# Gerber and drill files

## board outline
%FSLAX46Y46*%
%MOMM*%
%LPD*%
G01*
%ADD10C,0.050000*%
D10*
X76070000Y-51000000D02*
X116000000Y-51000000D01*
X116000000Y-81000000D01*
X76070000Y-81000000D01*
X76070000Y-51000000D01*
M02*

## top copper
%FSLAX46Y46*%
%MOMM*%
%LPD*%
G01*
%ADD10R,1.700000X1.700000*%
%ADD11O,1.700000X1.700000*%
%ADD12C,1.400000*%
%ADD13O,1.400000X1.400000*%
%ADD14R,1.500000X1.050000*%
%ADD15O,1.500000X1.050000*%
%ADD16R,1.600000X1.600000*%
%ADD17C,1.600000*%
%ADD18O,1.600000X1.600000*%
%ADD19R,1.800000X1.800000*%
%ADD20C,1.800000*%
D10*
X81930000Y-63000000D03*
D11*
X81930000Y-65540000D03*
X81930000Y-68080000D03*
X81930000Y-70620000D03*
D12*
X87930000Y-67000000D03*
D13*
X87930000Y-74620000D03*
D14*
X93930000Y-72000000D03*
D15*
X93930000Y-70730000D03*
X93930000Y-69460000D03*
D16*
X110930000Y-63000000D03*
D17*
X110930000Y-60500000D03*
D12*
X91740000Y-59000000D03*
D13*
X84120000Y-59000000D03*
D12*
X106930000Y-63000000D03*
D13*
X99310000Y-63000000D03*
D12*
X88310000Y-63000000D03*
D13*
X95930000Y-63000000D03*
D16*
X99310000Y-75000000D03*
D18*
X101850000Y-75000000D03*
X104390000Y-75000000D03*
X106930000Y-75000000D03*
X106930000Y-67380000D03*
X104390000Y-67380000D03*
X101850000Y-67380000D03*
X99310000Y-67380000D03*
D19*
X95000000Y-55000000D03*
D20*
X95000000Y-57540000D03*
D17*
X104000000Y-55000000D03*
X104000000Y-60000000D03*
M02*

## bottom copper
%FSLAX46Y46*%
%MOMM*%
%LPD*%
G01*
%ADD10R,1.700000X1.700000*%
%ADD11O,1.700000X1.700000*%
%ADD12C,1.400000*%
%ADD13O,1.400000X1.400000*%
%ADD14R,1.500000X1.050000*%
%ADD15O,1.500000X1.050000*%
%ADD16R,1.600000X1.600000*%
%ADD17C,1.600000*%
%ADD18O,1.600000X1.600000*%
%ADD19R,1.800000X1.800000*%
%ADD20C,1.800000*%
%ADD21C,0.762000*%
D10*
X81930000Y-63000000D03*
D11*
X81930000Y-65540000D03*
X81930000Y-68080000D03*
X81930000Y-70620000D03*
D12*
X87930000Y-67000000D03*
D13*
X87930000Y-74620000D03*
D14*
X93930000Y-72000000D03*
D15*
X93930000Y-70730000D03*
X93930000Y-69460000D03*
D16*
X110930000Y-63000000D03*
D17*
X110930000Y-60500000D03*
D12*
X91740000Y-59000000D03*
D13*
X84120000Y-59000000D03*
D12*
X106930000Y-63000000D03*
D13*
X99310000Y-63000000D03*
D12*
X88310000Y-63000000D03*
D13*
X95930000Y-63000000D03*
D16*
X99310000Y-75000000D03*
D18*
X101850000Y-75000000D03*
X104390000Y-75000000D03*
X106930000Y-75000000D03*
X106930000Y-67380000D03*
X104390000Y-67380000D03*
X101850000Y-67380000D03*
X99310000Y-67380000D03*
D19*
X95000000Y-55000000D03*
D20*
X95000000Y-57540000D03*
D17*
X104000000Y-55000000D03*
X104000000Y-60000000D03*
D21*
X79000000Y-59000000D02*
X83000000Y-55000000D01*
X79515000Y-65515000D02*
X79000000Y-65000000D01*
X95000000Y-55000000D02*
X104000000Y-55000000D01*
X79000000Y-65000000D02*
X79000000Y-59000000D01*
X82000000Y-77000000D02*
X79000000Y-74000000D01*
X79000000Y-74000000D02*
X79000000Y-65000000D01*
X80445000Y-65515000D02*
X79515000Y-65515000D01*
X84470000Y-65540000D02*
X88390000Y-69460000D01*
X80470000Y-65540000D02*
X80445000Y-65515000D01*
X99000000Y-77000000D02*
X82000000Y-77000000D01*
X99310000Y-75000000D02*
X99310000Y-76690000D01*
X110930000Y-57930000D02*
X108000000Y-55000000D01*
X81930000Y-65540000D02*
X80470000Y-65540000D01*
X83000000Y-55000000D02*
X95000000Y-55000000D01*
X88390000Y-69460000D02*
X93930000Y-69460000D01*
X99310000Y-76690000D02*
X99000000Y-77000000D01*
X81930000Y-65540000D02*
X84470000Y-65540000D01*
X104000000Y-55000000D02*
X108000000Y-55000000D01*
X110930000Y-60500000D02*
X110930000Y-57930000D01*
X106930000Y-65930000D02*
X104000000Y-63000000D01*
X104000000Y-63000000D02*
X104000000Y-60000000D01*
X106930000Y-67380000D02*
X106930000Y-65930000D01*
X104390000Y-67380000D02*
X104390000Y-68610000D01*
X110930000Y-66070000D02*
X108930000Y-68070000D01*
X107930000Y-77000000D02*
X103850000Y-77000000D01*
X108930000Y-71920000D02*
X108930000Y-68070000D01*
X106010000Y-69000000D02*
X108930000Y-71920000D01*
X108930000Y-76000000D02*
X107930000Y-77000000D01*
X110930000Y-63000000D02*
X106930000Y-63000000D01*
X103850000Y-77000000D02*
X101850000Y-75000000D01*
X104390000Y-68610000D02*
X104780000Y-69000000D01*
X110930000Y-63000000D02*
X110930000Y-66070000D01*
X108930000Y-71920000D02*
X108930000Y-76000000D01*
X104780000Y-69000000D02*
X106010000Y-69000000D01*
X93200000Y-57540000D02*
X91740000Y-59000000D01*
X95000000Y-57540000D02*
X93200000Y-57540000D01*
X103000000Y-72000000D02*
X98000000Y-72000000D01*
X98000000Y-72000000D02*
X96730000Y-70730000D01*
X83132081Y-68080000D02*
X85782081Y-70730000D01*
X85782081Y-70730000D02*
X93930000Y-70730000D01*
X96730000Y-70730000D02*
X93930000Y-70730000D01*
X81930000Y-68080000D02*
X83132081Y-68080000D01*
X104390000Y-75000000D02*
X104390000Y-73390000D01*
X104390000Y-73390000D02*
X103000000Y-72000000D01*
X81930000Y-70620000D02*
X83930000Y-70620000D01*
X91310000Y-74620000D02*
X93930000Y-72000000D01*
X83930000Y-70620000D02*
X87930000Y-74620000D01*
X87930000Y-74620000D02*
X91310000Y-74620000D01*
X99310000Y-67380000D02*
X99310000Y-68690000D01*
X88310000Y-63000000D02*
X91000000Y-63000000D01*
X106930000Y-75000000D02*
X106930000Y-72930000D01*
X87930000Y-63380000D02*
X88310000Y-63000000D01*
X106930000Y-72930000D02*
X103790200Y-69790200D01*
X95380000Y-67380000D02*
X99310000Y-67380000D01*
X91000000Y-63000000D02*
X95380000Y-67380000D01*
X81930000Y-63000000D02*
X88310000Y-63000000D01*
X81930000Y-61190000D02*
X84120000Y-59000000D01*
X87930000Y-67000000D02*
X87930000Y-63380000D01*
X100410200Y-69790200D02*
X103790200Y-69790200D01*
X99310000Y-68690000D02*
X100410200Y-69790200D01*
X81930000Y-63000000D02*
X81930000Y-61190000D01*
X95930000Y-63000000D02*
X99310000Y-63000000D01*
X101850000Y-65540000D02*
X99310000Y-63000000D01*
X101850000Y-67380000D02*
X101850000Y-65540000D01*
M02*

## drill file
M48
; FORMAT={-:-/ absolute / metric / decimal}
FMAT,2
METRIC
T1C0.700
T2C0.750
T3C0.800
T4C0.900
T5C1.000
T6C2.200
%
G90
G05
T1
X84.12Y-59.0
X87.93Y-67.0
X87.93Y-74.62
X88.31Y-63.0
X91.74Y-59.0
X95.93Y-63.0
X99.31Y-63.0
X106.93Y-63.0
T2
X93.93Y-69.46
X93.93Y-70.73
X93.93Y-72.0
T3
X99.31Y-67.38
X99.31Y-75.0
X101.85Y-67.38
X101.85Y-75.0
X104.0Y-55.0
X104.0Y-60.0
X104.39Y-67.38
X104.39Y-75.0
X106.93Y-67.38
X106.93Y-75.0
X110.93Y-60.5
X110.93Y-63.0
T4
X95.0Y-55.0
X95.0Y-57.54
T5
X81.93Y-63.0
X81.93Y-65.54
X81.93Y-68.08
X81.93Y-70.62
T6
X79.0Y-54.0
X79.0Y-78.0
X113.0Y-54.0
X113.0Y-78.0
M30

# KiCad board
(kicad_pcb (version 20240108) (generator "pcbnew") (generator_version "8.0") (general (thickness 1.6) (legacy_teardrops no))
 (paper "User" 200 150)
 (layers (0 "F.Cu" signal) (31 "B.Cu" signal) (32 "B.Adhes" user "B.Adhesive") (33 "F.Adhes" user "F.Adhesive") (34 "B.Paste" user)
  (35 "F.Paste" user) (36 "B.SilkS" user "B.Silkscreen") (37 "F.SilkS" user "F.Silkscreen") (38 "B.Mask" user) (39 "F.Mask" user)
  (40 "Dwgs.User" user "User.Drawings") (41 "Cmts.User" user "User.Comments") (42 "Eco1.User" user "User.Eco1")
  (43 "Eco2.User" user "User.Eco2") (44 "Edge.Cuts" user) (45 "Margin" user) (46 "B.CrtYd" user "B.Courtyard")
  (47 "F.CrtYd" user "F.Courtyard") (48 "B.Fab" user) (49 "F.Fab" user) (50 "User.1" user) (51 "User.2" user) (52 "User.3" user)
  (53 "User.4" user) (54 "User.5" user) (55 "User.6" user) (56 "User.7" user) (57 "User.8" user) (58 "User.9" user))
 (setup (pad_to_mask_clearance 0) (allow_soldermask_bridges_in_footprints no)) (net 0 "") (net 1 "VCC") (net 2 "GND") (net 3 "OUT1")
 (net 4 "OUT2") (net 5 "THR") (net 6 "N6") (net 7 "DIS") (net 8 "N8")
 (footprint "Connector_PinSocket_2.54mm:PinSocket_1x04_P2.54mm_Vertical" (layer "F.Cu") (at 81.93 63)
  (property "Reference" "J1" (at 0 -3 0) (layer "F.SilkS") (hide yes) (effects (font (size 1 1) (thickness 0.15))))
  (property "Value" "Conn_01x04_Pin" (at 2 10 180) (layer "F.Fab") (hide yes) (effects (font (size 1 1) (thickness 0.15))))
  (pad "1" thru_hole rect (at 0 0) (size 1.7 1.7) (drill 1) (layers "*.Cu" "*.Mask") (remove_unused_layers no) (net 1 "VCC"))
  (pad "2" thru_hole oval (at 0 2.54) (size 1.7 1.7) (drill 1) (layers "*.Cu" "*.Mask") (remove_unused_layers no) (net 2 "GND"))
  (pad "3" thru_hole oval (at 0 5.08) (size 1.7 1.7) (drill 1) (layers "*.Cu" "*.Mask") (remove_unused_layers no) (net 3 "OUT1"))
  (pad "4" thru_hole oval (at 0 7.62) (size 1.7 1.7) (drill 1) (layers "*.Cu" "*.Mask") (remove_unused_layers no) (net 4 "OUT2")))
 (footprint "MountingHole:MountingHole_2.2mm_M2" (layer "F.Cu") (at 113 54)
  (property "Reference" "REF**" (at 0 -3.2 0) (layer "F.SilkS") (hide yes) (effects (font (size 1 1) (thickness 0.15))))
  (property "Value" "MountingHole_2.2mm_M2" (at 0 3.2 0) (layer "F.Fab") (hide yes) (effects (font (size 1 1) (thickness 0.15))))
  (pad "" np_thru_hole circle (at 0 0) (size 2.2 2.2) (drill 2.2) (layers "*.Cu" "*.Mask")))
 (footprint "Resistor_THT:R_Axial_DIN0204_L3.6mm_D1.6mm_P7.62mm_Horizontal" (layer "F.Cu") (at 87.93 67 -90)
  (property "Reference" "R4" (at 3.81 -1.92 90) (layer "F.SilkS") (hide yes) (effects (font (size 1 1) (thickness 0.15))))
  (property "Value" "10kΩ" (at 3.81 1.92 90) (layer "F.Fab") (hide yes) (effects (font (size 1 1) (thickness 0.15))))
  (pad "1" thru_hole circle (at 0 0 270) (size 1.4 1.4) (drill 0.7) (layers "*.Cu" "*.Mask") (remove_unused_layers no) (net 1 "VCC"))
  (pad "2" thru_hole oval (at 7.62 0 270) (size 1.4 1.4) (drill 0.7) (layers "*.Cu" "*.Mask") (remove_unused_layers no) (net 4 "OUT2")))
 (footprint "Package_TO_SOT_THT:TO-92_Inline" (layer "F.Cu") (at 93.93 72 90)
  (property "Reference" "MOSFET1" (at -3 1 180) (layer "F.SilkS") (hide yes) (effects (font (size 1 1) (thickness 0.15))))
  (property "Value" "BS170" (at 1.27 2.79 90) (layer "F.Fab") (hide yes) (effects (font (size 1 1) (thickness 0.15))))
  (pad "1" thru_hole rect (at 0 0 90) (size 1.05 1.5) (drill 0.75) (layers "*.Cu" "*.Mask") (remove_unused_layers no) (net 4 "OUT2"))
  (pad "2" thru_hole oval (at 1.27 0 90) (size 1.05 1.5) (drill 0.75) (layers "*.Cu" "*.Mask") (remove_unused_layers no) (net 3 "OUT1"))
  (pad "3" thru_hole oval (at 2.54 0 90) (size 1.05 1.5) (drill 0.75) (layers "*.Cu" "*.Mask") (remove_unused_layers no) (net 2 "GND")))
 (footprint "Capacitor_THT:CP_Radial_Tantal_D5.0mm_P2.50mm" (layer "F.Cu") (at 110.93 63 90)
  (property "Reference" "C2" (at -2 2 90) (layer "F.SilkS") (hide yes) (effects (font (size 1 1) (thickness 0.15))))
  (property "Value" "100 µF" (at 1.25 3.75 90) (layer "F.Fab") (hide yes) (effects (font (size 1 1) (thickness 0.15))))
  (pad "1" thru_hole rect (at 0 0 90) (size 1.6 1.6) (drill 0.8) (layers "*.Cu" "*.Mask") (remove_unused_layers no) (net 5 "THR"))
  (pad "2" thru_hole circle (at 2.5 0 90) (size 1.6 1.6) (drill 0.8) (layers "*.Cu" "*.Mask") (remove_unused_layers no) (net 2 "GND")))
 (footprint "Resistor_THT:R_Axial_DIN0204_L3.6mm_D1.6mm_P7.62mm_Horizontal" (layer "F.Cu") (at 91.74 59 180)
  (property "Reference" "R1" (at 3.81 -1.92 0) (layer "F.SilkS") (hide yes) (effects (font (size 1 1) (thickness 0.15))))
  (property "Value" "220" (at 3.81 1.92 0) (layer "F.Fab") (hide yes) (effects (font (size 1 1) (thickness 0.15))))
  (pad "1" thru_hole circle (at 0 0 180) (size 1.4 1.4) (drill 0.7) (layers "*.Cu" "*.Mask") (remove_unused_layers no) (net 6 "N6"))
  (pad "2" thru_hole oval (at 7.62 0 180) (size 1.4 1.4) (drill 0.7) (layers "*.Cu" "*.Mask") (remove_unused_layers no) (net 1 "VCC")))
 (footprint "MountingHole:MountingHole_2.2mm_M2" (layer "F.Cu") (at 113 78)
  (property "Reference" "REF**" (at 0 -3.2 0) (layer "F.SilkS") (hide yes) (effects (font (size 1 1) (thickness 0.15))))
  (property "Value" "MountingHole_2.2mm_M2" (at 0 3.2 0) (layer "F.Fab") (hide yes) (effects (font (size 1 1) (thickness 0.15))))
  (pad "" np_thru_hole circle (at 0 0) (size 2.2 2.2) (drill 2.2) (layers "*.Cu" "*.Mask")))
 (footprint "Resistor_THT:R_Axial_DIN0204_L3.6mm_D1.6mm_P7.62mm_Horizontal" (layer "F.Cu") (at 106.93 63 180)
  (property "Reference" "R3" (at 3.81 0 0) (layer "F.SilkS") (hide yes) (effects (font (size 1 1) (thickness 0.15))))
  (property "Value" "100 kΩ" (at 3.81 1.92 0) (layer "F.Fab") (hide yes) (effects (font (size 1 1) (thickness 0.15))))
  (pad "1" thru_hole circle (at 0 0 180) (size 1.4 1.4) (drill 0.7) (layers "*.Cu" "*.Mask") (remove_unused_layers no) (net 5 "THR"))
  (pad "2" thru_hole oval (at 7.62 0 180) (size 1.4 1.4) (drill 0.7) (layers "*.Cu" "*.Mask") (remove_unused_layers no) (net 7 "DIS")))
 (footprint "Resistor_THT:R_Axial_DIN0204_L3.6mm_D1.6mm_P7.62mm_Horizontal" (layer "F.Cu") (at 88.31 63)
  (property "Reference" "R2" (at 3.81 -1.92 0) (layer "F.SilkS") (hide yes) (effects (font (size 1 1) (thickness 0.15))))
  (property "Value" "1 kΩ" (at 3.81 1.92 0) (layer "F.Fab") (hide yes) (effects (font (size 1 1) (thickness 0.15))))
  (pad "1" thru_hole circle (at 0 0) (size 1.4 1.4) (drill 0.7) (layers "*.Cu" "*.Mask") (remove_unused_layers no) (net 1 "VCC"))
  (pad "2" thru_hole oval (at 7.62 0) (size 1.4 1.4) (drill 0.7) (layers "*.Cu" "*.Mask") (remove_unused_layers no) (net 7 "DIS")))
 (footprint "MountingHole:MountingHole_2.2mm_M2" (layer "F.Cu") (at 79 78)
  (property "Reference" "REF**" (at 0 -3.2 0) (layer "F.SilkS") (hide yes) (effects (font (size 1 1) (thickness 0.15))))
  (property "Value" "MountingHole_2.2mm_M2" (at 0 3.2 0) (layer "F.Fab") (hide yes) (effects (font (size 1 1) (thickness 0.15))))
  (pad "" np_thru_hole circle (at 0 0) (size 2.2 2.2) (drill 2.2) (layers "*.Cu" "*.Mask")))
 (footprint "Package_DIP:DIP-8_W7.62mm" (layer "F.Cu") (at 99.31 75 90)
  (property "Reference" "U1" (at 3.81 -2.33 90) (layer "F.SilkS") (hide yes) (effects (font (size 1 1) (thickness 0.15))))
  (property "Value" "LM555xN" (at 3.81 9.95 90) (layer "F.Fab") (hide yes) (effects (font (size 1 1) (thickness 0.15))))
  (pad "1" thru_hole rect (at 0 0 90) (size 1.6 1.6) (drill 0.8) (layers "*.Cu" "*.Mask") (remove_unused_layers no) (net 2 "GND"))
  (pad "2" thru_hole oval (at 0 2.54 90) (size 1.6 1.6) (drill 0.8) (layers "*.Cu" "*.Mask") (remove_unused_layers no) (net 5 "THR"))
  (pad "3" thru_hole oval (at 0 5.08 90) (size 1.6 1.6) (drill 0.8) (layers "*.Cu" "*.Mask") (remove_unused_layers no) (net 3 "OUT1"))
  (pad "4" thru_hole oval (at 0 7.62 90) (size 1.6 1.6) (drill 0.8) (layers "*.Cu" "*.Mask") (remove_unused_layers no) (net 1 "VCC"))
  (pad "5" thru_hole oval (at 7.62 7.62 90) (size 1.6 1.6) (drill 0.8) (layers "*.Cu" "*.Mask") (remove_unused_layers no) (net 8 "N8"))
  (pad "6" thru_hole oval (at 7.62 5.08 90) (size 1.6 1.6) (drill 0.8) (layers "*.Cu" "*.Mask") (remove_unused_layers no) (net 5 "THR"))
  (pad "7" thru_hole oval (at 7.62 2.54 90) (size 1.6 1.6) (drill 0.8) (layers "*.Cu" "*.Mask") (remove_unused_layers no) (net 7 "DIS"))
  (pad "8" thru_hole oval (at 7.62 0 90) (size 1.6 1.6) (drill 0.8) (layers "*.Cu" "*.Mask") (remove_unused_layers no) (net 1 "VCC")))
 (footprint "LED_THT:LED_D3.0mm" (layer "F.Cu") (at 95 55 -90)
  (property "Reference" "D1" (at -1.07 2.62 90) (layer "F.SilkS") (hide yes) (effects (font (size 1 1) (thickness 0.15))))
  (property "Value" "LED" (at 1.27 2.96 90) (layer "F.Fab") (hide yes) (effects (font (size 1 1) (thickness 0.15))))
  (pad "1" thru_hole rect (at 0 0 270) (size 1.8 1.8) (drill 0.9) (layers "*.Cu" "*.Mask") (remove_unused_layers no) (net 2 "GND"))
  (pad "2" thru_hole circle (at 2.54 0 270) (size 1.8 1.8) (drill 0.9) (layers "*.Cu" "*.Mask") (remove_unused_layers no) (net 6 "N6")))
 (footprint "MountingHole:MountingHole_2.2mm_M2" (layer "F.Cu") (at 79 54)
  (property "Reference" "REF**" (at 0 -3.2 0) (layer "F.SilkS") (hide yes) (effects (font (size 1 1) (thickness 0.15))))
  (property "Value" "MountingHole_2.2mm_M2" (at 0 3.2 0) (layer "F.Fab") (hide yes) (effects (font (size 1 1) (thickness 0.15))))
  (pad "" np_thru_hole circle (at 0 0) (size 2.2 2.2) (drill 2.2) (layers "*.Cu" "*.Mask")))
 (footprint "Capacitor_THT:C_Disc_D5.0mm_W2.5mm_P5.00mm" (layer "F.Cu") (at 104 55 -90)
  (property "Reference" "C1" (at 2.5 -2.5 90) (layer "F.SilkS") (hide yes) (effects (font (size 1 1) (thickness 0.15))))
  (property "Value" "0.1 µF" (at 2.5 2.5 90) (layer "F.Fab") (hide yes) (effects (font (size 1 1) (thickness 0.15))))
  (pad "1" thru_hole circle (at 0 0 270) (size 1.6 1.6) (drill 0.8) (layers "*.Cu" "*.Mask") (remove_unused_layers no) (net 2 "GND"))
  (pad "2" thru_hole circle (at 5 0 270) (size 1.6 1.6) (drill 0.8) (layers "*.Cu" "*.Mask") (remove_unused_layers no) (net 8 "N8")))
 (gr_rect (start 76.07 51) (end 116 81) (stroke (width 0.05) (type default)) (fill none) (layer "Edge.Cuts"))
 (segment (start 79 59) (end 83 55) (width 0.762) (layer "B.Cu") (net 2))
 (segment (start 79.515 65.515) (end 79 65) (width 0.762) (layer "B.Cu") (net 2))
 (segment (start 95 55) (end 104 55) (width 0.762) (layer "B.Cu") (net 2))
 (segment (start 79 65) (end 79 59) (width 0.762) (layer "B.Cu") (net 2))
 (segment (start 82 77) (end 79 74) (width 0.762) (layer "B.Cu") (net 2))
 (segment (start 79 74) (end 79 65) (width 0.762) (layer "B.Cu") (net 2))
 (segment (start 80.445 65.515) (end 79.515 65.515) (width 0.762) (layer "B.Cu") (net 2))
 (segment (start 84.47 65.54) (end 88.39 69.46) (width 0.762) (layer "B.Cu") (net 2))
 (segment (start 80.47 65.54) (end 80.445 65.515) (width 0.762) (layer "B.Cu") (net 2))
 (segment (start 99 77) (end 82 77) (width 0.762) (layer "B.Cu") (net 2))
 (segment (start 99.31 75) (end 99.31 76.69) (width 0.762) (layer "B.Cu") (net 2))
 (segment (start 110.93 57.93) (end 108 55) (width 0.762) (layer "B.Cu") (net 2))
 (segment (start 81.93 65.54) (end 80.47 65.54) (width 0.762) (layer "B.Cu") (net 2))
 (segment (start 83 55) (end 95 55) (width 0.762) (layer "B.Cu") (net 2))
 (segment (start 88.39 69.46) (end 93.93 69.46) (width 0.762) (layer "B.Cu") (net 2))
 (segment (start 99.31 76.69) (end 99 77) (width 0.762) (layer "B.Cu") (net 2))
 (segment (start 81.93 65.54) (end 84.47 65.54) (width 0.762) (layer "B.Cu") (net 2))
 (segment (start 104 55) (end 108 55) (width 0.762) (layer "B.Cu") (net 2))
 (segment (start 110.93 60.5) (end 110.93 57.93) (width 0.762) (layer "B.Cu") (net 2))
 (segment (start 106.93 65.93) (end 104 63) (width 0.762) (layer "B.Cu") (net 8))
 (segment (start 104 63) (end 104 60) (width 0.762) (layer "B.Cu") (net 8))
 (segment (start 106.93 67.38) (end 106.93 65.93) (width 0.762) (layer "B.Cu") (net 8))
 (segment (start 104.39 67.38) (end 104.39 68.61) (width 0.762) (layer "B.Cu") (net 5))
 (segment (start 110.93 66.07) (end 108.93 68.07) (width 0.762) (layer "B.Cu") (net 5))
 (segment (start 107.93 77) (end 103.85 77) (width 0.762) (layer "B.Cu") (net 5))
 (segment (start 108.93 71.92) (end 108.93 68.07) (width 0.762) (layer "B.Cu") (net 5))
 (segment (start 106.01 69) (end 108.93 71.92) (width 0.762) (layer "B.Cu") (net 5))
 (segment (start 108.93 76) (end 107.93 77) (width 0.762) (layer "B.Cu") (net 5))
 (segment (start 110.93 63) (end 106.93 63) (width 0.762) (layer "B.Cu") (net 5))
 (segment (start 103.85 77) (end 101.85 75) (width 0.762) (layer "B.Cu") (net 5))
 (segment (start 104.39 68.61) (end 104.78 69) (width 0.762) (layer "B.Cu") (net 5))
 (segment (start 110.93 63) (end 110.93 66.07) (width 0.762) (layer "B.Cu") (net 5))
 (segment (start 108.93 71.92) (end 108.93 76) (width 0.762) (layer "B.Cu") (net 5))
 (segment (start 104.78 69) (end 106.01 69) (width 0.762) (layer "B.Cu") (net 5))
 (segment (start 93.2 57.54) (end 91.74 59) (width 0.762) (layer "B.Cu") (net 6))
 (segment (start 95 57.54) (end 93.2 57.54) (width 0.762) (layer "B.Cu") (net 6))
 (segment (start 103 72) (end 98 72) (width 0.762) (layer "B.Cu") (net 3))
 (segment (start 98 72) (end 96.73 70.73) (width 0.762) (layer "B.Cu") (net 3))
 (segment (start 83.132081 68.08) (end 85.782081 70.73) (width 0.762) (layer "B.Cu") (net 3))
 (segment (start 85.782081 70.73) (end 93.93 70.73) (width 0.762) (layer "B.Cu") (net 3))
 (segment (start 96.73 70.73) (end 93.93 70.73) (width 0.762) (layer "B.Cu") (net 3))
 (segment (start 81.93 68.08) (end 83.132081 68.08) (width 0.762) (layer "B.Cu") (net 3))
 (segment (start 104.39 75) (end 104.39 73.39) (width 0.762) (layer "B.Cu") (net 3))
 (segment (start 104.39 73.39) (end 103 72) (width 0.762) (layer "B.Cu") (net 3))
 (segment (start 81.93 70.62) (end 83.93 70.62) (width 0.762) (layer "B.Cu") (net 4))
 (segment (start 91.31 74.62) (end 93.93 72) (width 0.762) (layer "B.Cu") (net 4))
 (segment (start 83.93 70.62) (end 87.93 74.62) (width 0.762) (layer "B.Cu") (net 4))
 (segment (start 87.93 74.62) (end 91.31 74.62) (width 0.762) (layer "B.Cu") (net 4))
 (segment (start 99.31 67.38) (end 99.31 68.69) (width 0.762) (layer "B.Cu") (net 1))
 (segment (start 88.31 63) (end 91 63) (width 0.762) (layer "B.Cu") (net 1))
 (segment (start 106.93 75) (end 106.93 72.93) (width 0.762) (layer "B.Cu") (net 1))
 (segment (start 87.93 63.38) (end 88.31 63) (width 0.762) (layer "B.Cu") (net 1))
 (segment (start 106.93 72.93) (end 103.7902 69.7902) (width 0.762) (layer "B.Cu") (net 1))
 (segment (start 95.38 67.38) (end 99.31 67.38) (width 0.762) (layer "B.Cu") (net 1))
 (segment (start 91 63) (end 95.38 67.38) (width 0.762) (layer "B.Cu") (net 1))
 (segment (start 81.93 63) (end 88.31 63) (width 0.762) (layer "B.Cu") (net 1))
 (segment (start 81.93 61.19) (end 84.12 59) (width 0.762) (layer "B.Cu") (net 1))
 (segment (start 87.93 67) (end 87.93 63.38) (width 0.762) (layer "B.Cu") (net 1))
 (segment (start 100.4102 69.7902) (end 103.7902 69.7902) (width 0.762) (layer "B.Cu") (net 1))
 (segment (start 99.31 68.69) (end 100.4102 69.7902) (width 0.762) (layer "B.Cu") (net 1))
 (segment (start 81.93 63) (end 81.93 61.19) (width 0.762) (layer "B.Cu") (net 1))
 (segment (start 95.93 63) (end 99.31 63) (width 0.762) (layer "B.Cu") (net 7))
 (segment (start 101.85 65.54) (end 99.31 63) (width 0.762) (layer "B.Cu") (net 7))
 (segment (start 101.85 67.38) (end 101.85 65.54) (width 0.762) (layer "B.Cu") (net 7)))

